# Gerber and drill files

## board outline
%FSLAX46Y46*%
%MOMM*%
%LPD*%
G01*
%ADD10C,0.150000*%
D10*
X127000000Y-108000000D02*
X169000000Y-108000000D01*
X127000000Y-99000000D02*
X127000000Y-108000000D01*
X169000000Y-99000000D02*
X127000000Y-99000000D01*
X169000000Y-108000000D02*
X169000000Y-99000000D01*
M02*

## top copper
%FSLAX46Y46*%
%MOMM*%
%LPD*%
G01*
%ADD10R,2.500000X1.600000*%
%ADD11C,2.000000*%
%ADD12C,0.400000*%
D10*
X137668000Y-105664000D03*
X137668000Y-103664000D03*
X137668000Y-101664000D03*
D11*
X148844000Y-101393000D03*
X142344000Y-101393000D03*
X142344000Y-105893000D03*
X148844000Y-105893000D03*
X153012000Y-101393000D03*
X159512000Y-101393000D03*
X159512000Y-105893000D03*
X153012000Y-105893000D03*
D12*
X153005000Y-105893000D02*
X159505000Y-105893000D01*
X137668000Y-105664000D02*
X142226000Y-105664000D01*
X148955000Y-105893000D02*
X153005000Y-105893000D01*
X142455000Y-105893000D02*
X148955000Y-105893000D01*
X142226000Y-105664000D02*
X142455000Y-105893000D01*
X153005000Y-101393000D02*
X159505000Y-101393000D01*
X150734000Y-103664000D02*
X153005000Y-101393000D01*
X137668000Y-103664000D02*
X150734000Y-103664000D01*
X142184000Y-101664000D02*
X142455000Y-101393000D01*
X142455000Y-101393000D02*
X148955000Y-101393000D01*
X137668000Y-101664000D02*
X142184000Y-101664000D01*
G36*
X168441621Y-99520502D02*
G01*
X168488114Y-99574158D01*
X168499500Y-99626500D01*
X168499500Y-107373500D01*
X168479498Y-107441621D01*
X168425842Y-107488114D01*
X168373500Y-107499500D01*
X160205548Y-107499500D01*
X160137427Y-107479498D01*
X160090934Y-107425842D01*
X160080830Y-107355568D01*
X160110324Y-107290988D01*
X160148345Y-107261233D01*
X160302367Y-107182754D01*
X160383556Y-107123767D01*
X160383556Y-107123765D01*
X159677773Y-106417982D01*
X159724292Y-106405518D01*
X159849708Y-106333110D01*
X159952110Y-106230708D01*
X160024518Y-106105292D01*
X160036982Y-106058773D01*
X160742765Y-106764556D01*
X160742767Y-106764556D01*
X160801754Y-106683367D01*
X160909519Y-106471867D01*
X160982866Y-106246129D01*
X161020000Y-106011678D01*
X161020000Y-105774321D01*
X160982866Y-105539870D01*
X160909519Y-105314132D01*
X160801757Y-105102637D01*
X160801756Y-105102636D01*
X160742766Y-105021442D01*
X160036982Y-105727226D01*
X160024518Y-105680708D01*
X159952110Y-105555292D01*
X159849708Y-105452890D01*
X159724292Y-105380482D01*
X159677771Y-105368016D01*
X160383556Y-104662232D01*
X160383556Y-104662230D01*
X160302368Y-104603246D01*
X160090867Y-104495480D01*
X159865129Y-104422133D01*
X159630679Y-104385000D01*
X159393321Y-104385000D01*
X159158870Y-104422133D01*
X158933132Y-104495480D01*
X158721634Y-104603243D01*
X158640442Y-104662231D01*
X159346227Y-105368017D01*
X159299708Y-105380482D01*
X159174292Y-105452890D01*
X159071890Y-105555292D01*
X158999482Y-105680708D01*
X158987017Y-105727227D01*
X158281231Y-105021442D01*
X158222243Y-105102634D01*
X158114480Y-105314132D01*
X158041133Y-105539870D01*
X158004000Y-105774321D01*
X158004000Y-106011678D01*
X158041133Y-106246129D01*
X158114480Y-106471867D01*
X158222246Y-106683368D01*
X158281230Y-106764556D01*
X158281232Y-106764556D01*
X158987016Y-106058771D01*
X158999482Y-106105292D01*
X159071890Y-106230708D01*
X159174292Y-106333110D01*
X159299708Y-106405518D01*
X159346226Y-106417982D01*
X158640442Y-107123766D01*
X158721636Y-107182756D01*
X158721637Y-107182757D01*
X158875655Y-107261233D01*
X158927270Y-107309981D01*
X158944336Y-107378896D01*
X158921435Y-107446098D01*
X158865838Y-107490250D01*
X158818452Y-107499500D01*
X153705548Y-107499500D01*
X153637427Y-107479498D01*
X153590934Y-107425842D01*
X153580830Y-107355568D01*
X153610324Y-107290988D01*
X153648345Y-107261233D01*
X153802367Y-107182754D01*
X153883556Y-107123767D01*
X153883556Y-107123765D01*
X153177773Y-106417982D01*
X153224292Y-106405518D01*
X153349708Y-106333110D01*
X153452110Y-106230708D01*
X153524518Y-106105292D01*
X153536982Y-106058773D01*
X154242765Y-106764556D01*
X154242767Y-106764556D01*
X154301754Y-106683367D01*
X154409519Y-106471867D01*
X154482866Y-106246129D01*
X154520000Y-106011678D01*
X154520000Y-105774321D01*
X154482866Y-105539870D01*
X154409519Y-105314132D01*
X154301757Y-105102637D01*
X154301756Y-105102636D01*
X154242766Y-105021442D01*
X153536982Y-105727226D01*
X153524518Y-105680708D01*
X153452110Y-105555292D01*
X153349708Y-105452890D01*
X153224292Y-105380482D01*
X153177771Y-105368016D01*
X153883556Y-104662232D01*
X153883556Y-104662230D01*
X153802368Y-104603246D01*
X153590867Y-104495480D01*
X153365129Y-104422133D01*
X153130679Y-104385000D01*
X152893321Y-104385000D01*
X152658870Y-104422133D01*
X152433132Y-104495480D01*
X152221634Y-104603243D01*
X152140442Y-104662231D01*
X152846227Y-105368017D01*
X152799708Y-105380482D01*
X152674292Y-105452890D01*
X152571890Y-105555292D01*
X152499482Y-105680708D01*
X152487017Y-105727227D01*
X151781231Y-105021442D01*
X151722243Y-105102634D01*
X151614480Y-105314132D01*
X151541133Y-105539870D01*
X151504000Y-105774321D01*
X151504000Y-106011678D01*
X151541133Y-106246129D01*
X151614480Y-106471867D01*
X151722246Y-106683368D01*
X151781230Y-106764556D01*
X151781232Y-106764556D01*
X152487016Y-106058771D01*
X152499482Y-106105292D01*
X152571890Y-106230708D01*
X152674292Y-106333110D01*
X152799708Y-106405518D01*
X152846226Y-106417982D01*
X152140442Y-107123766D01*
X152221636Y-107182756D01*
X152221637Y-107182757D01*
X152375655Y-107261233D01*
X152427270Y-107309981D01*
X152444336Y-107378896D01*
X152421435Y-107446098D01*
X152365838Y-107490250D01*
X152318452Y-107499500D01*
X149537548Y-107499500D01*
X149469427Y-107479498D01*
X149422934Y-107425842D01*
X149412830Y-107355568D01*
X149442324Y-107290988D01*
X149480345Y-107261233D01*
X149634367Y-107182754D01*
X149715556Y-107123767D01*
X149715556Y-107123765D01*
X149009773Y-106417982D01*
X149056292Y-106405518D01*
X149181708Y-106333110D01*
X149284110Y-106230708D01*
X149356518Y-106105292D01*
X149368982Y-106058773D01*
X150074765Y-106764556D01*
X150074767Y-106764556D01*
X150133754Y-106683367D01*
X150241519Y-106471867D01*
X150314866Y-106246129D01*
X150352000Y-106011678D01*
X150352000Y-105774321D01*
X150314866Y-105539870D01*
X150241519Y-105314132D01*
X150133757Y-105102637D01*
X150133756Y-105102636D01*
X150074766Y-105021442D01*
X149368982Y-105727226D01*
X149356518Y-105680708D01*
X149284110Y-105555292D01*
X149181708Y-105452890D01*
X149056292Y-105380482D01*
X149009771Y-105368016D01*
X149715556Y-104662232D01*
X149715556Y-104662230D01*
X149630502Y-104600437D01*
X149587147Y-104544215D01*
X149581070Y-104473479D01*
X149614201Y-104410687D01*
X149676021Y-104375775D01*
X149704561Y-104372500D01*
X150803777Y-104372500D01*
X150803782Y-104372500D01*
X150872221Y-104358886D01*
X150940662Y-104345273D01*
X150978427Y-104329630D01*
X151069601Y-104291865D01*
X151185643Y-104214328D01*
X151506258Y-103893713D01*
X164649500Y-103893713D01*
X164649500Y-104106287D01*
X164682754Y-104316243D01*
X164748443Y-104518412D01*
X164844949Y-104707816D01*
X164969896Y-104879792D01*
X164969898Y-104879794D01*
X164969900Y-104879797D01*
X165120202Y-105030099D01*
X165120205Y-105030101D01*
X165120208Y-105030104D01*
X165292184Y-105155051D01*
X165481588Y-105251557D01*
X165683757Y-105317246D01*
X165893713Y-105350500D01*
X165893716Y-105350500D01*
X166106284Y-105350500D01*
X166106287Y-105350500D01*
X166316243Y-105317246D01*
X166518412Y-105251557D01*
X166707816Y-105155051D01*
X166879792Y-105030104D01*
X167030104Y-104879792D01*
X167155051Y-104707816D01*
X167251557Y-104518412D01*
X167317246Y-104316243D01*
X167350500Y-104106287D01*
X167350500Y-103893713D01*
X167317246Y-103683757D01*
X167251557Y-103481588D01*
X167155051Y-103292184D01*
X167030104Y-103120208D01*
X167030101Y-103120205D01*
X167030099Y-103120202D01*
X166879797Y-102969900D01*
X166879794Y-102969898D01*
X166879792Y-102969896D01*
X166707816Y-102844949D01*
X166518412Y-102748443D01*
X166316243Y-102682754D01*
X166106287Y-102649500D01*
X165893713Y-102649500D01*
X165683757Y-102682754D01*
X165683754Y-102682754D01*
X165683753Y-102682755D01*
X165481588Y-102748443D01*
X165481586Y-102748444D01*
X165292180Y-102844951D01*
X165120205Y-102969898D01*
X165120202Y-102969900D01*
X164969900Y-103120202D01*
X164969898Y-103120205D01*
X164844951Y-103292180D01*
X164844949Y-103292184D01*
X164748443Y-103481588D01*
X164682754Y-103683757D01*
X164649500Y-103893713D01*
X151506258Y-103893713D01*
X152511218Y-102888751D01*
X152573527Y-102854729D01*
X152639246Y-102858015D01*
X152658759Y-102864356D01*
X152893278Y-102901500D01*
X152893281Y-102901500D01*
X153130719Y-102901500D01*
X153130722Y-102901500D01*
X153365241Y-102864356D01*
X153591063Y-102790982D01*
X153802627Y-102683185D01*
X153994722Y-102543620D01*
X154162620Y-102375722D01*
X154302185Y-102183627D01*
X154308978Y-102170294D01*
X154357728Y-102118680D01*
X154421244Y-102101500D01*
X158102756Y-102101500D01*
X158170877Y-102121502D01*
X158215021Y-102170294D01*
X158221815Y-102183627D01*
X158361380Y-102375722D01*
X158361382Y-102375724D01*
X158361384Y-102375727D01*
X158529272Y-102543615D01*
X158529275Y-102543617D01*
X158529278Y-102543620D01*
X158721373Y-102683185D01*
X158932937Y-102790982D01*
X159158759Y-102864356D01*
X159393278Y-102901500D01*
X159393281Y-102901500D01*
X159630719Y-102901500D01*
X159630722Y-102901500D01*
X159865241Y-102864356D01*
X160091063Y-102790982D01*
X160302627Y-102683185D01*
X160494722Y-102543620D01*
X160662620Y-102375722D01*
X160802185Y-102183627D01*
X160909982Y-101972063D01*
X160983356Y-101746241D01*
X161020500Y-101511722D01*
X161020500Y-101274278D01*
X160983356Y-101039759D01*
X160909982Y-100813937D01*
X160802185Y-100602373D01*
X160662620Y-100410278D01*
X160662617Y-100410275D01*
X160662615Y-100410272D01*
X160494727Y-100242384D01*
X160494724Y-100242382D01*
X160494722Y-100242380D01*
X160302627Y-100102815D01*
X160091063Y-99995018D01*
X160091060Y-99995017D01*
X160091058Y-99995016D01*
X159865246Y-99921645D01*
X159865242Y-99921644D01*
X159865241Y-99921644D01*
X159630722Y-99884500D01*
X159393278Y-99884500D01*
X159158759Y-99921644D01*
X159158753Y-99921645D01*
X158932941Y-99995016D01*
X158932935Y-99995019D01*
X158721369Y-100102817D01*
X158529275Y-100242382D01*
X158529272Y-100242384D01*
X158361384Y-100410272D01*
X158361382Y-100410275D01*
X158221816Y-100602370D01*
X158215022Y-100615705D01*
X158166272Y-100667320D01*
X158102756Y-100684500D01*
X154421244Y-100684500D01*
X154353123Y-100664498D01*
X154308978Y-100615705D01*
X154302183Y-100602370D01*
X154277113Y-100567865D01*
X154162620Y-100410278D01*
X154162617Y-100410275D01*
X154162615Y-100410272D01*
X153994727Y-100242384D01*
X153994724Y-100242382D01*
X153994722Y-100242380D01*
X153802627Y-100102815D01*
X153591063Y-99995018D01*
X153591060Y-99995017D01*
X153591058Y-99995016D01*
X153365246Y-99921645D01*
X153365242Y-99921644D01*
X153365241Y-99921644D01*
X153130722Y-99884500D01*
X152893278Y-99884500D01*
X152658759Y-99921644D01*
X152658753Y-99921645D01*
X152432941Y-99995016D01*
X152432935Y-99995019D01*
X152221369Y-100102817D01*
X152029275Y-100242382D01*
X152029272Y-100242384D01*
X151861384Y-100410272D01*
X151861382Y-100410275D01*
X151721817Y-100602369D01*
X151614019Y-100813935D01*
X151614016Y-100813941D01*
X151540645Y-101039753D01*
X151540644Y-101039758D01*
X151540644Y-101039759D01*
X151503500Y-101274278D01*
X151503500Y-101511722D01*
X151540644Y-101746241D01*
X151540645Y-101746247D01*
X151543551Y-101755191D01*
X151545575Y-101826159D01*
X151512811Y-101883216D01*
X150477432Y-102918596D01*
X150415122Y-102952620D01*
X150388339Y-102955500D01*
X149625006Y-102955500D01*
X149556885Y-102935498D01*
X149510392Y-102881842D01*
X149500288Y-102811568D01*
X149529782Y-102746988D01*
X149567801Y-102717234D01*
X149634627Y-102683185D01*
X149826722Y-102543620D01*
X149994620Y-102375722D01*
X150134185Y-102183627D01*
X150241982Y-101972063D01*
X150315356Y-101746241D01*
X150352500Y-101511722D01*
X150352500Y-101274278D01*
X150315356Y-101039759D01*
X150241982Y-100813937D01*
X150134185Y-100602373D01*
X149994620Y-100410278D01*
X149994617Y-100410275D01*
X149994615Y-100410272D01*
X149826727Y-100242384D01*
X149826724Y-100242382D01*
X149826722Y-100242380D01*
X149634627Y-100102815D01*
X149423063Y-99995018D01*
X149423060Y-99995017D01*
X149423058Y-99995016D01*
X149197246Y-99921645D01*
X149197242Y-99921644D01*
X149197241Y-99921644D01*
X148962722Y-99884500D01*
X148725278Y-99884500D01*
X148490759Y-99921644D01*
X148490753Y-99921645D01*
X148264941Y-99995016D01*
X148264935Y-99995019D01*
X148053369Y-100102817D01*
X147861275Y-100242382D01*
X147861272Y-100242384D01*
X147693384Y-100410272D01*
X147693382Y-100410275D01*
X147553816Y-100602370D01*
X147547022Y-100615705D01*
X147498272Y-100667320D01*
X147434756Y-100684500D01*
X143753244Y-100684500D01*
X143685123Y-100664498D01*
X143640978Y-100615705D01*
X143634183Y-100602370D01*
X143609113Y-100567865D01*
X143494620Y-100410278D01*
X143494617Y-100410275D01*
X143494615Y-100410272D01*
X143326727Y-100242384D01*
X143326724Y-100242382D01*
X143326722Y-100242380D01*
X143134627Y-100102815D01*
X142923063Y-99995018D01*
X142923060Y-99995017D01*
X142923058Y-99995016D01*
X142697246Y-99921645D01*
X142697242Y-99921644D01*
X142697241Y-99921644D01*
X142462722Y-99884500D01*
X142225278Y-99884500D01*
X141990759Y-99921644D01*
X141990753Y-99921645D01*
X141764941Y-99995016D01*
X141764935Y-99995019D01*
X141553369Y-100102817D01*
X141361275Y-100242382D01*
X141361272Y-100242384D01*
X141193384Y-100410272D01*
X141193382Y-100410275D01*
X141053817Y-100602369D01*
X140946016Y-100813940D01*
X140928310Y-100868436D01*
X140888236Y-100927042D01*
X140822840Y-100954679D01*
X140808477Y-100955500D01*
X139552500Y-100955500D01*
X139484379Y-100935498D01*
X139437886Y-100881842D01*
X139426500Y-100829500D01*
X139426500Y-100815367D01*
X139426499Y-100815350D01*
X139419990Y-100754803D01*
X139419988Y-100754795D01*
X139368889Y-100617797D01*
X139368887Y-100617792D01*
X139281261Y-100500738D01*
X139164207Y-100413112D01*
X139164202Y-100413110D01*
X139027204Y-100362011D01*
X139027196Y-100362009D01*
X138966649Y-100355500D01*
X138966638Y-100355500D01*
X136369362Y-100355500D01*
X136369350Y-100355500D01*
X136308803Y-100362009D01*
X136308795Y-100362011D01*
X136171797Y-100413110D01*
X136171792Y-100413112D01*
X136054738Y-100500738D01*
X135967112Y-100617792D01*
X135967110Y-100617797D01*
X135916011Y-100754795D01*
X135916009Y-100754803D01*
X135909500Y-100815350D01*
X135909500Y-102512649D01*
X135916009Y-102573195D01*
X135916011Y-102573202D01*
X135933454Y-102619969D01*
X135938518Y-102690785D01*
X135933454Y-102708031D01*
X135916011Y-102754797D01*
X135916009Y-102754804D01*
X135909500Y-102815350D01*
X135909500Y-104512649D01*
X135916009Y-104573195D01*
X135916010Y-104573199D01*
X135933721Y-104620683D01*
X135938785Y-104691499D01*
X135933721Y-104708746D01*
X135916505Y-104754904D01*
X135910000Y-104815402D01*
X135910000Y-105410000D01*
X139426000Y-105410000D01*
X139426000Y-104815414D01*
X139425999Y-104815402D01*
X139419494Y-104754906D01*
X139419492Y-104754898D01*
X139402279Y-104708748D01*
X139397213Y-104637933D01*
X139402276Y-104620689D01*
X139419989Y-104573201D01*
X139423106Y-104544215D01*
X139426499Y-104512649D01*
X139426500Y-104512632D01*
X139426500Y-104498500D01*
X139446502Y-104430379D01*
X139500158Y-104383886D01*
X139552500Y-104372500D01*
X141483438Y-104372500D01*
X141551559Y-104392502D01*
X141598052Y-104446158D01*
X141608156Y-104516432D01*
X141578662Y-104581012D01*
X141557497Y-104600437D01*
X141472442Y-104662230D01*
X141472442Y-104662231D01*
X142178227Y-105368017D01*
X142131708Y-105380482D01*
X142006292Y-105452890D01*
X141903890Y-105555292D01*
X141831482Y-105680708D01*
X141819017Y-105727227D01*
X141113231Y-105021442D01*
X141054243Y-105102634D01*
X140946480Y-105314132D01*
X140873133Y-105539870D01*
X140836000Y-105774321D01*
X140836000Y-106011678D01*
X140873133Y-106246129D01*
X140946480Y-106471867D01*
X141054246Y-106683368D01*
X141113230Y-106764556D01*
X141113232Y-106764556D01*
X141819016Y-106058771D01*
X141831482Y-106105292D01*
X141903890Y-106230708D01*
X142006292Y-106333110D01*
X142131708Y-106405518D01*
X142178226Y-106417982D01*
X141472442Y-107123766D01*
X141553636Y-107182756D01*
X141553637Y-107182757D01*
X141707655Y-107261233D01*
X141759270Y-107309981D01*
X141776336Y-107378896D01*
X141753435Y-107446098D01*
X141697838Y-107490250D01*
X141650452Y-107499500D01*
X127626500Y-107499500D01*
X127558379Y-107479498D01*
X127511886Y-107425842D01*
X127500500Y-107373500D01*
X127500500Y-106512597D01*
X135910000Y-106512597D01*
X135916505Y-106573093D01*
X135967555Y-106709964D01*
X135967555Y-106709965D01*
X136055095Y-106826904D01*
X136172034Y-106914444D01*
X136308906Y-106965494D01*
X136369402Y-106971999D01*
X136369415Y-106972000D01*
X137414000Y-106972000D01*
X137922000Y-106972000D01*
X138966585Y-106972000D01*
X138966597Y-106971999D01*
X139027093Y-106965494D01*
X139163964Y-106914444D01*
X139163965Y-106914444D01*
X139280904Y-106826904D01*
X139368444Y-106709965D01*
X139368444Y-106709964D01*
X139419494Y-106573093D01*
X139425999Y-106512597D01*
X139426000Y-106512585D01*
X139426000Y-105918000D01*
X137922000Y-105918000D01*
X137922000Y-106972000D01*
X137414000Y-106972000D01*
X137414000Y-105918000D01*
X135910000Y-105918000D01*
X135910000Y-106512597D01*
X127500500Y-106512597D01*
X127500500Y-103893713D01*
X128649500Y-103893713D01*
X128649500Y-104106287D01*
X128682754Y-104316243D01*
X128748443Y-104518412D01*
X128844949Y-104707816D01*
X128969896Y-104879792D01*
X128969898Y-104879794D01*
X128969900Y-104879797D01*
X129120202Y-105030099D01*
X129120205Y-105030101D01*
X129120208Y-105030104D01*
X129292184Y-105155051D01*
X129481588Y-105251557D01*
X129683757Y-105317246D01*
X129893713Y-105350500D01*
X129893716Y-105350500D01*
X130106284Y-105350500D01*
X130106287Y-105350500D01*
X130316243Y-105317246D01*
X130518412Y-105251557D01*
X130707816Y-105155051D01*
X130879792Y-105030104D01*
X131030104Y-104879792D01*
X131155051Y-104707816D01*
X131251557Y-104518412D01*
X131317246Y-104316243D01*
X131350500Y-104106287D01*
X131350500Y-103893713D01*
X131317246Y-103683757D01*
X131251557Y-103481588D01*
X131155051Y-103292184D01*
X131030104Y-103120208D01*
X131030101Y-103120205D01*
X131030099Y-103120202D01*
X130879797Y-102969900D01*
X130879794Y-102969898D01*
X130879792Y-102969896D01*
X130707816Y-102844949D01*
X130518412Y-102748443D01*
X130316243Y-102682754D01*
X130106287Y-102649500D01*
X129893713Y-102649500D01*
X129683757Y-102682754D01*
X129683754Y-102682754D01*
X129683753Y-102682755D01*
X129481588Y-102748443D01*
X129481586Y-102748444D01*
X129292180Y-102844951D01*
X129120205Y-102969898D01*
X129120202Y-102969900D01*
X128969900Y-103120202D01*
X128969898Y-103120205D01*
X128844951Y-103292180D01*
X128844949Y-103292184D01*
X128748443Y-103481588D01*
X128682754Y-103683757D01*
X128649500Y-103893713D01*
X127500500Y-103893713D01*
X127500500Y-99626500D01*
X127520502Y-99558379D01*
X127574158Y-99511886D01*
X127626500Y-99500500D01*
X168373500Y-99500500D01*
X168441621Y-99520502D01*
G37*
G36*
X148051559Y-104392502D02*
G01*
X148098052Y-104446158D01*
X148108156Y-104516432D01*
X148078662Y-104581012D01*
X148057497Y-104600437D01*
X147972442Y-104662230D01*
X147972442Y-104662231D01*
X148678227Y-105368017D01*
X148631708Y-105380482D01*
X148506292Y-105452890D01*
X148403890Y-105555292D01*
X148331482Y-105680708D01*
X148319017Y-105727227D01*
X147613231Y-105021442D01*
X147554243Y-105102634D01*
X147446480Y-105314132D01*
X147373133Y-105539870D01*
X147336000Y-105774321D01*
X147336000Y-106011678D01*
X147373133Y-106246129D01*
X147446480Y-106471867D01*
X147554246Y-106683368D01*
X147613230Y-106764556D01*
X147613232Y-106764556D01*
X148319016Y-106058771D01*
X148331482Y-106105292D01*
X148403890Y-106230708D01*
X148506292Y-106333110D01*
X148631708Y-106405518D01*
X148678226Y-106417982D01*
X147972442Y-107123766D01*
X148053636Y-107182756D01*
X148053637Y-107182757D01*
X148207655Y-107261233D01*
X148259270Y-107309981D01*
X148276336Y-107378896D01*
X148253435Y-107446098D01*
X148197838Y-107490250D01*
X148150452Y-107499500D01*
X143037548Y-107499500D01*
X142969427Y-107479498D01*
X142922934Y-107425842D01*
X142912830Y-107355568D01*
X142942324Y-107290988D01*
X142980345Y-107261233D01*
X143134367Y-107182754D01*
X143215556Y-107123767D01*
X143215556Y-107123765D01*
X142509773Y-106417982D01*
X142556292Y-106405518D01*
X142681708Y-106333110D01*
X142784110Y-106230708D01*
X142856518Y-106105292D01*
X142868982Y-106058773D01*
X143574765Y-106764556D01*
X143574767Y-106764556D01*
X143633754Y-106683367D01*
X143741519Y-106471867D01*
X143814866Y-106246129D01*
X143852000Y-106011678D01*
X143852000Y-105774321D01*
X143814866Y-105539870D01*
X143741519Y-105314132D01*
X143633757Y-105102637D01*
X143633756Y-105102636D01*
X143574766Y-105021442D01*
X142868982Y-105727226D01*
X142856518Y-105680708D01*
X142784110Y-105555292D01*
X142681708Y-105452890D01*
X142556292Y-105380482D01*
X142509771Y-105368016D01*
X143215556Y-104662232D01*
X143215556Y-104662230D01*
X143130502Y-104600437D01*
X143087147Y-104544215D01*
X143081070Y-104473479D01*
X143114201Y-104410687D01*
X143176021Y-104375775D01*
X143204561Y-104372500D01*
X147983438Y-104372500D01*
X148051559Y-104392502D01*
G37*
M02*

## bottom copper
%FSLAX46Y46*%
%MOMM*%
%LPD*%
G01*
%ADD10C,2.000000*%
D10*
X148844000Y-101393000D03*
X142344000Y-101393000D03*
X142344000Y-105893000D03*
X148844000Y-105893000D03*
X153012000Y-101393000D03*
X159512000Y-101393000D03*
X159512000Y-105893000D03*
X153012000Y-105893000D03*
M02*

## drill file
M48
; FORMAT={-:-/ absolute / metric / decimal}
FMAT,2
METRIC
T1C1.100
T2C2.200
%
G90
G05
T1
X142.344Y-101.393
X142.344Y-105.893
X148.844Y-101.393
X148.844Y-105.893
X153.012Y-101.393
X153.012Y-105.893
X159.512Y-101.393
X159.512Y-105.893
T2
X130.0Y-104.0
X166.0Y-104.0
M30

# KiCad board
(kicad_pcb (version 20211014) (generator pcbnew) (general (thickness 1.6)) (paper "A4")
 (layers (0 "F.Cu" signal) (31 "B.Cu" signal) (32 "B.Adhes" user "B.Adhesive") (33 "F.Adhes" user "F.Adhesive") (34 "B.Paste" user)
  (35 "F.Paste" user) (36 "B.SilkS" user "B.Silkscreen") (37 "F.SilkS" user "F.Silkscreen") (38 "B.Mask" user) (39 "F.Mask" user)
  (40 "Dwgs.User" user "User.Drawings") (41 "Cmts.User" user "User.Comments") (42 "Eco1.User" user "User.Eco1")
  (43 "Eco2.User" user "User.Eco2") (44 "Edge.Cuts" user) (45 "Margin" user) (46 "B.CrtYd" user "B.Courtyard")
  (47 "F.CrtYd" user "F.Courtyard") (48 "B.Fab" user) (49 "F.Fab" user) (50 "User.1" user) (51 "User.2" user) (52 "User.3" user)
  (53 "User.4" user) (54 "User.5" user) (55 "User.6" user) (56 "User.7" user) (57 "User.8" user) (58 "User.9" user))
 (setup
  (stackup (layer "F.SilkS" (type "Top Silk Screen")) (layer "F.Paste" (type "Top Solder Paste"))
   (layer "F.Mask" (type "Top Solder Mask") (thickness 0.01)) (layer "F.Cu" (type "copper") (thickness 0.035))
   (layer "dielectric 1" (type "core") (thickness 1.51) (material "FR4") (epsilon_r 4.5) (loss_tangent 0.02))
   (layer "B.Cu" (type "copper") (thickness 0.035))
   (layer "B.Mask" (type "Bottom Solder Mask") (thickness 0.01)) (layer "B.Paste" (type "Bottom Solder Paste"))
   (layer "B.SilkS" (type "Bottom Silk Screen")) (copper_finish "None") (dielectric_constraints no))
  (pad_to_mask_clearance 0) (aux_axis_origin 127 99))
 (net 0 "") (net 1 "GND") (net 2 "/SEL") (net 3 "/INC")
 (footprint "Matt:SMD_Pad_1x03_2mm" (layer "F.Cu") (at 137.668 105.664 90)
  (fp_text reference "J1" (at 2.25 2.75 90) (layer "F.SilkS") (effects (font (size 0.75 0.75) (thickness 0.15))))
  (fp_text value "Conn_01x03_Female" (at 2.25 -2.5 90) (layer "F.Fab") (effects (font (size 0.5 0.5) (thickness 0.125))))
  (pad "1" smd rect (at 0 0 90) (size 1.6 2.5) (layers "F.Cu" "F.Paste" "F.Mask") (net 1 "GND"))
  (pad "2" smd rect (at 2 0 90) (size 1.6 2.5) (layers "F.Cu" "F.Paste" "F.Mask") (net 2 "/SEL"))
  (pad "3" smd rect (at 4 0 90) (size 1.6 2.5) (layers "F.Cu" "F.Paste" "F.Mask") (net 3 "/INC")))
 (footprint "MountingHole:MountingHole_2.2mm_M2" (layer "F.Cu") (at 130 104)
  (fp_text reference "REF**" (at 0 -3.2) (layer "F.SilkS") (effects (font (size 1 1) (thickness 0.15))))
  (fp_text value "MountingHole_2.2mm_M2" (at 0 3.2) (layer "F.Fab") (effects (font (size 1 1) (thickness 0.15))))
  (pad "" np_thru_hole circle (at 0 0) (size 2.2 2.2) (drill 2.2) (layers *.Cu *.Mask)))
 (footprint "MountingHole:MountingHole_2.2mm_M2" (layer "F.Cu") (at 166 104)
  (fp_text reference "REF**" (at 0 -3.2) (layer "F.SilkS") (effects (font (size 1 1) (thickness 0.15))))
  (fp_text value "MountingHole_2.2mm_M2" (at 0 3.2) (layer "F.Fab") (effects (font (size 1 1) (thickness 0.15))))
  (pad "" np_thru_hole circle (at 0 0) (size 2.2 2.2) (drill 2.2) (layers *.Cu *.Mask)))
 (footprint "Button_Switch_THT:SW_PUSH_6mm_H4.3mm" (layer "B.Cu") (at 148.844 101.393 180)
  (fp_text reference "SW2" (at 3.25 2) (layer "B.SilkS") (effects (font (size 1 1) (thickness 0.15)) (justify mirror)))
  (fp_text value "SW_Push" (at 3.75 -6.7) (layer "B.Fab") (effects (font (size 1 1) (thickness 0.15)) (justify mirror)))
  (pad "1" thru_hole circle (at 0 0 90) (size 2 2) (drill 1.1) (layers *.Cu *.Mask) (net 3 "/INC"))
  (pad "1" thru_hole circle (at 6.5 0 90) (size 2 2) (drill 1.1) (layers *.Cu *.Mask) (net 3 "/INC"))
  (pad "2" thru_hole circle (at 6.5 -4.5 90) (size 2 2) (drill 1.1) (layers *.Cu *.Mask) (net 1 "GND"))
  (pad "2" thru_hole circle (at 0 -4.5 90) (size 2 2) (drill 1.1) (layers *.Cu *.Mask) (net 1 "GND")))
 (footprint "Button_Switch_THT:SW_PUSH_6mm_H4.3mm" (layer "B.Cu") (at 159.512 101.393 180)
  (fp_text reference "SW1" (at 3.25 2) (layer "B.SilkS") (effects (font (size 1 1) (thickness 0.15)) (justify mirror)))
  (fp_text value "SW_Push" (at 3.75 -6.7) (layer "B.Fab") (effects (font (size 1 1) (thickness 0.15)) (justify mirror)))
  (pad "1" thru_hole circle (at 6.5 0 90) (size 2 2) (drill 1.1) (layers *.Cu *.Mask) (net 2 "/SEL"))
  (pad "1" thru_hole circle (at 0 0 90) (size 2 2) (drill 1.1) (layers *.Cu *.Mask) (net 2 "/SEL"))
  (pad "2" thru_hole circle (at 0 -4.5 90) (size 2 2) (drill 1.1) (layers *.Cu *.Mask) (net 1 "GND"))
  (pad "2" thru_hole circle (at 6.5 -4.5 90) (size 2 2) (drill 1.1) (layers *.Cu *.Mask) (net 1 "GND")))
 (gr_line (start 127 108) (end 169 108) (layer "Edge.Cuts") (width 0.15))
 (gr_line (start 127 99) (end 127 108) (layer "Edge.Cuts") (width 0.15))
 (gr_line (start 169 99) (end 127 99) (layer "Edge.Cuts") (width 0.15))
 (gr_line (start 169 108) (end 169 99) (layer "Edge.Cuts") (width 0.15))
 (segment (start 153.005 105.893) (end 159.505 105.893) (width 0.4) (layer "F.Cu") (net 1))
 (segment (start 137.668 105.664) (end 142.226 105.664) (width 0.4) (layer "F.Cu") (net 1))
 (segment (start 148.955 105.893) (end 153.005 105.893) (width 0.4) (layer "F.Cu") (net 1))
 (segment (start 142.455 105.893) (end 148.955 105.893) (width 0.4) (layer "F.Cu") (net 1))
 (segment (start 142.226 105.664) (end 142.455 105.893) (width 0.4) (layer "F.Cu") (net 1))
 (segment (start 153.005 101.393) (end 159.505 101.393) (width 0.4) (layer "F.Cu") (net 2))
 (segment (start 150.734 103.664) (end 153.005 101.393) (width 0.4) (layer "F.Cu") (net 2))
 (segment (start 137.668 103.664) (end 150.734 103.664) (width 0.4) (layer "F.Cu") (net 2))
 (segment (start 142.184 101.664) (end 142.455 101.393) (width 0.4) (layer "F.Cu") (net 3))
 (segment (start 142.455 101.393) (end 148.955 101.393) (width 0.4) (layer "F.Cu") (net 3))
 (segment (start 137.668 101.664) (end 142.184 101.664) (width 0.4) (layer "F.Cu") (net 3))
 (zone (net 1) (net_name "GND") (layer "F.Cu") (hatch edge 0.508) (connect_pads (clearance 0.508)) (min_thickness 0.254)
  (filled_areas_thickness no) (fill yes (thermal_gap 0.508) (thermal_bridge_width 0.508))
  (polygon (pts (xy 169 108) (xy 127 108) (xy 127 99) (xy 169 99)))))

